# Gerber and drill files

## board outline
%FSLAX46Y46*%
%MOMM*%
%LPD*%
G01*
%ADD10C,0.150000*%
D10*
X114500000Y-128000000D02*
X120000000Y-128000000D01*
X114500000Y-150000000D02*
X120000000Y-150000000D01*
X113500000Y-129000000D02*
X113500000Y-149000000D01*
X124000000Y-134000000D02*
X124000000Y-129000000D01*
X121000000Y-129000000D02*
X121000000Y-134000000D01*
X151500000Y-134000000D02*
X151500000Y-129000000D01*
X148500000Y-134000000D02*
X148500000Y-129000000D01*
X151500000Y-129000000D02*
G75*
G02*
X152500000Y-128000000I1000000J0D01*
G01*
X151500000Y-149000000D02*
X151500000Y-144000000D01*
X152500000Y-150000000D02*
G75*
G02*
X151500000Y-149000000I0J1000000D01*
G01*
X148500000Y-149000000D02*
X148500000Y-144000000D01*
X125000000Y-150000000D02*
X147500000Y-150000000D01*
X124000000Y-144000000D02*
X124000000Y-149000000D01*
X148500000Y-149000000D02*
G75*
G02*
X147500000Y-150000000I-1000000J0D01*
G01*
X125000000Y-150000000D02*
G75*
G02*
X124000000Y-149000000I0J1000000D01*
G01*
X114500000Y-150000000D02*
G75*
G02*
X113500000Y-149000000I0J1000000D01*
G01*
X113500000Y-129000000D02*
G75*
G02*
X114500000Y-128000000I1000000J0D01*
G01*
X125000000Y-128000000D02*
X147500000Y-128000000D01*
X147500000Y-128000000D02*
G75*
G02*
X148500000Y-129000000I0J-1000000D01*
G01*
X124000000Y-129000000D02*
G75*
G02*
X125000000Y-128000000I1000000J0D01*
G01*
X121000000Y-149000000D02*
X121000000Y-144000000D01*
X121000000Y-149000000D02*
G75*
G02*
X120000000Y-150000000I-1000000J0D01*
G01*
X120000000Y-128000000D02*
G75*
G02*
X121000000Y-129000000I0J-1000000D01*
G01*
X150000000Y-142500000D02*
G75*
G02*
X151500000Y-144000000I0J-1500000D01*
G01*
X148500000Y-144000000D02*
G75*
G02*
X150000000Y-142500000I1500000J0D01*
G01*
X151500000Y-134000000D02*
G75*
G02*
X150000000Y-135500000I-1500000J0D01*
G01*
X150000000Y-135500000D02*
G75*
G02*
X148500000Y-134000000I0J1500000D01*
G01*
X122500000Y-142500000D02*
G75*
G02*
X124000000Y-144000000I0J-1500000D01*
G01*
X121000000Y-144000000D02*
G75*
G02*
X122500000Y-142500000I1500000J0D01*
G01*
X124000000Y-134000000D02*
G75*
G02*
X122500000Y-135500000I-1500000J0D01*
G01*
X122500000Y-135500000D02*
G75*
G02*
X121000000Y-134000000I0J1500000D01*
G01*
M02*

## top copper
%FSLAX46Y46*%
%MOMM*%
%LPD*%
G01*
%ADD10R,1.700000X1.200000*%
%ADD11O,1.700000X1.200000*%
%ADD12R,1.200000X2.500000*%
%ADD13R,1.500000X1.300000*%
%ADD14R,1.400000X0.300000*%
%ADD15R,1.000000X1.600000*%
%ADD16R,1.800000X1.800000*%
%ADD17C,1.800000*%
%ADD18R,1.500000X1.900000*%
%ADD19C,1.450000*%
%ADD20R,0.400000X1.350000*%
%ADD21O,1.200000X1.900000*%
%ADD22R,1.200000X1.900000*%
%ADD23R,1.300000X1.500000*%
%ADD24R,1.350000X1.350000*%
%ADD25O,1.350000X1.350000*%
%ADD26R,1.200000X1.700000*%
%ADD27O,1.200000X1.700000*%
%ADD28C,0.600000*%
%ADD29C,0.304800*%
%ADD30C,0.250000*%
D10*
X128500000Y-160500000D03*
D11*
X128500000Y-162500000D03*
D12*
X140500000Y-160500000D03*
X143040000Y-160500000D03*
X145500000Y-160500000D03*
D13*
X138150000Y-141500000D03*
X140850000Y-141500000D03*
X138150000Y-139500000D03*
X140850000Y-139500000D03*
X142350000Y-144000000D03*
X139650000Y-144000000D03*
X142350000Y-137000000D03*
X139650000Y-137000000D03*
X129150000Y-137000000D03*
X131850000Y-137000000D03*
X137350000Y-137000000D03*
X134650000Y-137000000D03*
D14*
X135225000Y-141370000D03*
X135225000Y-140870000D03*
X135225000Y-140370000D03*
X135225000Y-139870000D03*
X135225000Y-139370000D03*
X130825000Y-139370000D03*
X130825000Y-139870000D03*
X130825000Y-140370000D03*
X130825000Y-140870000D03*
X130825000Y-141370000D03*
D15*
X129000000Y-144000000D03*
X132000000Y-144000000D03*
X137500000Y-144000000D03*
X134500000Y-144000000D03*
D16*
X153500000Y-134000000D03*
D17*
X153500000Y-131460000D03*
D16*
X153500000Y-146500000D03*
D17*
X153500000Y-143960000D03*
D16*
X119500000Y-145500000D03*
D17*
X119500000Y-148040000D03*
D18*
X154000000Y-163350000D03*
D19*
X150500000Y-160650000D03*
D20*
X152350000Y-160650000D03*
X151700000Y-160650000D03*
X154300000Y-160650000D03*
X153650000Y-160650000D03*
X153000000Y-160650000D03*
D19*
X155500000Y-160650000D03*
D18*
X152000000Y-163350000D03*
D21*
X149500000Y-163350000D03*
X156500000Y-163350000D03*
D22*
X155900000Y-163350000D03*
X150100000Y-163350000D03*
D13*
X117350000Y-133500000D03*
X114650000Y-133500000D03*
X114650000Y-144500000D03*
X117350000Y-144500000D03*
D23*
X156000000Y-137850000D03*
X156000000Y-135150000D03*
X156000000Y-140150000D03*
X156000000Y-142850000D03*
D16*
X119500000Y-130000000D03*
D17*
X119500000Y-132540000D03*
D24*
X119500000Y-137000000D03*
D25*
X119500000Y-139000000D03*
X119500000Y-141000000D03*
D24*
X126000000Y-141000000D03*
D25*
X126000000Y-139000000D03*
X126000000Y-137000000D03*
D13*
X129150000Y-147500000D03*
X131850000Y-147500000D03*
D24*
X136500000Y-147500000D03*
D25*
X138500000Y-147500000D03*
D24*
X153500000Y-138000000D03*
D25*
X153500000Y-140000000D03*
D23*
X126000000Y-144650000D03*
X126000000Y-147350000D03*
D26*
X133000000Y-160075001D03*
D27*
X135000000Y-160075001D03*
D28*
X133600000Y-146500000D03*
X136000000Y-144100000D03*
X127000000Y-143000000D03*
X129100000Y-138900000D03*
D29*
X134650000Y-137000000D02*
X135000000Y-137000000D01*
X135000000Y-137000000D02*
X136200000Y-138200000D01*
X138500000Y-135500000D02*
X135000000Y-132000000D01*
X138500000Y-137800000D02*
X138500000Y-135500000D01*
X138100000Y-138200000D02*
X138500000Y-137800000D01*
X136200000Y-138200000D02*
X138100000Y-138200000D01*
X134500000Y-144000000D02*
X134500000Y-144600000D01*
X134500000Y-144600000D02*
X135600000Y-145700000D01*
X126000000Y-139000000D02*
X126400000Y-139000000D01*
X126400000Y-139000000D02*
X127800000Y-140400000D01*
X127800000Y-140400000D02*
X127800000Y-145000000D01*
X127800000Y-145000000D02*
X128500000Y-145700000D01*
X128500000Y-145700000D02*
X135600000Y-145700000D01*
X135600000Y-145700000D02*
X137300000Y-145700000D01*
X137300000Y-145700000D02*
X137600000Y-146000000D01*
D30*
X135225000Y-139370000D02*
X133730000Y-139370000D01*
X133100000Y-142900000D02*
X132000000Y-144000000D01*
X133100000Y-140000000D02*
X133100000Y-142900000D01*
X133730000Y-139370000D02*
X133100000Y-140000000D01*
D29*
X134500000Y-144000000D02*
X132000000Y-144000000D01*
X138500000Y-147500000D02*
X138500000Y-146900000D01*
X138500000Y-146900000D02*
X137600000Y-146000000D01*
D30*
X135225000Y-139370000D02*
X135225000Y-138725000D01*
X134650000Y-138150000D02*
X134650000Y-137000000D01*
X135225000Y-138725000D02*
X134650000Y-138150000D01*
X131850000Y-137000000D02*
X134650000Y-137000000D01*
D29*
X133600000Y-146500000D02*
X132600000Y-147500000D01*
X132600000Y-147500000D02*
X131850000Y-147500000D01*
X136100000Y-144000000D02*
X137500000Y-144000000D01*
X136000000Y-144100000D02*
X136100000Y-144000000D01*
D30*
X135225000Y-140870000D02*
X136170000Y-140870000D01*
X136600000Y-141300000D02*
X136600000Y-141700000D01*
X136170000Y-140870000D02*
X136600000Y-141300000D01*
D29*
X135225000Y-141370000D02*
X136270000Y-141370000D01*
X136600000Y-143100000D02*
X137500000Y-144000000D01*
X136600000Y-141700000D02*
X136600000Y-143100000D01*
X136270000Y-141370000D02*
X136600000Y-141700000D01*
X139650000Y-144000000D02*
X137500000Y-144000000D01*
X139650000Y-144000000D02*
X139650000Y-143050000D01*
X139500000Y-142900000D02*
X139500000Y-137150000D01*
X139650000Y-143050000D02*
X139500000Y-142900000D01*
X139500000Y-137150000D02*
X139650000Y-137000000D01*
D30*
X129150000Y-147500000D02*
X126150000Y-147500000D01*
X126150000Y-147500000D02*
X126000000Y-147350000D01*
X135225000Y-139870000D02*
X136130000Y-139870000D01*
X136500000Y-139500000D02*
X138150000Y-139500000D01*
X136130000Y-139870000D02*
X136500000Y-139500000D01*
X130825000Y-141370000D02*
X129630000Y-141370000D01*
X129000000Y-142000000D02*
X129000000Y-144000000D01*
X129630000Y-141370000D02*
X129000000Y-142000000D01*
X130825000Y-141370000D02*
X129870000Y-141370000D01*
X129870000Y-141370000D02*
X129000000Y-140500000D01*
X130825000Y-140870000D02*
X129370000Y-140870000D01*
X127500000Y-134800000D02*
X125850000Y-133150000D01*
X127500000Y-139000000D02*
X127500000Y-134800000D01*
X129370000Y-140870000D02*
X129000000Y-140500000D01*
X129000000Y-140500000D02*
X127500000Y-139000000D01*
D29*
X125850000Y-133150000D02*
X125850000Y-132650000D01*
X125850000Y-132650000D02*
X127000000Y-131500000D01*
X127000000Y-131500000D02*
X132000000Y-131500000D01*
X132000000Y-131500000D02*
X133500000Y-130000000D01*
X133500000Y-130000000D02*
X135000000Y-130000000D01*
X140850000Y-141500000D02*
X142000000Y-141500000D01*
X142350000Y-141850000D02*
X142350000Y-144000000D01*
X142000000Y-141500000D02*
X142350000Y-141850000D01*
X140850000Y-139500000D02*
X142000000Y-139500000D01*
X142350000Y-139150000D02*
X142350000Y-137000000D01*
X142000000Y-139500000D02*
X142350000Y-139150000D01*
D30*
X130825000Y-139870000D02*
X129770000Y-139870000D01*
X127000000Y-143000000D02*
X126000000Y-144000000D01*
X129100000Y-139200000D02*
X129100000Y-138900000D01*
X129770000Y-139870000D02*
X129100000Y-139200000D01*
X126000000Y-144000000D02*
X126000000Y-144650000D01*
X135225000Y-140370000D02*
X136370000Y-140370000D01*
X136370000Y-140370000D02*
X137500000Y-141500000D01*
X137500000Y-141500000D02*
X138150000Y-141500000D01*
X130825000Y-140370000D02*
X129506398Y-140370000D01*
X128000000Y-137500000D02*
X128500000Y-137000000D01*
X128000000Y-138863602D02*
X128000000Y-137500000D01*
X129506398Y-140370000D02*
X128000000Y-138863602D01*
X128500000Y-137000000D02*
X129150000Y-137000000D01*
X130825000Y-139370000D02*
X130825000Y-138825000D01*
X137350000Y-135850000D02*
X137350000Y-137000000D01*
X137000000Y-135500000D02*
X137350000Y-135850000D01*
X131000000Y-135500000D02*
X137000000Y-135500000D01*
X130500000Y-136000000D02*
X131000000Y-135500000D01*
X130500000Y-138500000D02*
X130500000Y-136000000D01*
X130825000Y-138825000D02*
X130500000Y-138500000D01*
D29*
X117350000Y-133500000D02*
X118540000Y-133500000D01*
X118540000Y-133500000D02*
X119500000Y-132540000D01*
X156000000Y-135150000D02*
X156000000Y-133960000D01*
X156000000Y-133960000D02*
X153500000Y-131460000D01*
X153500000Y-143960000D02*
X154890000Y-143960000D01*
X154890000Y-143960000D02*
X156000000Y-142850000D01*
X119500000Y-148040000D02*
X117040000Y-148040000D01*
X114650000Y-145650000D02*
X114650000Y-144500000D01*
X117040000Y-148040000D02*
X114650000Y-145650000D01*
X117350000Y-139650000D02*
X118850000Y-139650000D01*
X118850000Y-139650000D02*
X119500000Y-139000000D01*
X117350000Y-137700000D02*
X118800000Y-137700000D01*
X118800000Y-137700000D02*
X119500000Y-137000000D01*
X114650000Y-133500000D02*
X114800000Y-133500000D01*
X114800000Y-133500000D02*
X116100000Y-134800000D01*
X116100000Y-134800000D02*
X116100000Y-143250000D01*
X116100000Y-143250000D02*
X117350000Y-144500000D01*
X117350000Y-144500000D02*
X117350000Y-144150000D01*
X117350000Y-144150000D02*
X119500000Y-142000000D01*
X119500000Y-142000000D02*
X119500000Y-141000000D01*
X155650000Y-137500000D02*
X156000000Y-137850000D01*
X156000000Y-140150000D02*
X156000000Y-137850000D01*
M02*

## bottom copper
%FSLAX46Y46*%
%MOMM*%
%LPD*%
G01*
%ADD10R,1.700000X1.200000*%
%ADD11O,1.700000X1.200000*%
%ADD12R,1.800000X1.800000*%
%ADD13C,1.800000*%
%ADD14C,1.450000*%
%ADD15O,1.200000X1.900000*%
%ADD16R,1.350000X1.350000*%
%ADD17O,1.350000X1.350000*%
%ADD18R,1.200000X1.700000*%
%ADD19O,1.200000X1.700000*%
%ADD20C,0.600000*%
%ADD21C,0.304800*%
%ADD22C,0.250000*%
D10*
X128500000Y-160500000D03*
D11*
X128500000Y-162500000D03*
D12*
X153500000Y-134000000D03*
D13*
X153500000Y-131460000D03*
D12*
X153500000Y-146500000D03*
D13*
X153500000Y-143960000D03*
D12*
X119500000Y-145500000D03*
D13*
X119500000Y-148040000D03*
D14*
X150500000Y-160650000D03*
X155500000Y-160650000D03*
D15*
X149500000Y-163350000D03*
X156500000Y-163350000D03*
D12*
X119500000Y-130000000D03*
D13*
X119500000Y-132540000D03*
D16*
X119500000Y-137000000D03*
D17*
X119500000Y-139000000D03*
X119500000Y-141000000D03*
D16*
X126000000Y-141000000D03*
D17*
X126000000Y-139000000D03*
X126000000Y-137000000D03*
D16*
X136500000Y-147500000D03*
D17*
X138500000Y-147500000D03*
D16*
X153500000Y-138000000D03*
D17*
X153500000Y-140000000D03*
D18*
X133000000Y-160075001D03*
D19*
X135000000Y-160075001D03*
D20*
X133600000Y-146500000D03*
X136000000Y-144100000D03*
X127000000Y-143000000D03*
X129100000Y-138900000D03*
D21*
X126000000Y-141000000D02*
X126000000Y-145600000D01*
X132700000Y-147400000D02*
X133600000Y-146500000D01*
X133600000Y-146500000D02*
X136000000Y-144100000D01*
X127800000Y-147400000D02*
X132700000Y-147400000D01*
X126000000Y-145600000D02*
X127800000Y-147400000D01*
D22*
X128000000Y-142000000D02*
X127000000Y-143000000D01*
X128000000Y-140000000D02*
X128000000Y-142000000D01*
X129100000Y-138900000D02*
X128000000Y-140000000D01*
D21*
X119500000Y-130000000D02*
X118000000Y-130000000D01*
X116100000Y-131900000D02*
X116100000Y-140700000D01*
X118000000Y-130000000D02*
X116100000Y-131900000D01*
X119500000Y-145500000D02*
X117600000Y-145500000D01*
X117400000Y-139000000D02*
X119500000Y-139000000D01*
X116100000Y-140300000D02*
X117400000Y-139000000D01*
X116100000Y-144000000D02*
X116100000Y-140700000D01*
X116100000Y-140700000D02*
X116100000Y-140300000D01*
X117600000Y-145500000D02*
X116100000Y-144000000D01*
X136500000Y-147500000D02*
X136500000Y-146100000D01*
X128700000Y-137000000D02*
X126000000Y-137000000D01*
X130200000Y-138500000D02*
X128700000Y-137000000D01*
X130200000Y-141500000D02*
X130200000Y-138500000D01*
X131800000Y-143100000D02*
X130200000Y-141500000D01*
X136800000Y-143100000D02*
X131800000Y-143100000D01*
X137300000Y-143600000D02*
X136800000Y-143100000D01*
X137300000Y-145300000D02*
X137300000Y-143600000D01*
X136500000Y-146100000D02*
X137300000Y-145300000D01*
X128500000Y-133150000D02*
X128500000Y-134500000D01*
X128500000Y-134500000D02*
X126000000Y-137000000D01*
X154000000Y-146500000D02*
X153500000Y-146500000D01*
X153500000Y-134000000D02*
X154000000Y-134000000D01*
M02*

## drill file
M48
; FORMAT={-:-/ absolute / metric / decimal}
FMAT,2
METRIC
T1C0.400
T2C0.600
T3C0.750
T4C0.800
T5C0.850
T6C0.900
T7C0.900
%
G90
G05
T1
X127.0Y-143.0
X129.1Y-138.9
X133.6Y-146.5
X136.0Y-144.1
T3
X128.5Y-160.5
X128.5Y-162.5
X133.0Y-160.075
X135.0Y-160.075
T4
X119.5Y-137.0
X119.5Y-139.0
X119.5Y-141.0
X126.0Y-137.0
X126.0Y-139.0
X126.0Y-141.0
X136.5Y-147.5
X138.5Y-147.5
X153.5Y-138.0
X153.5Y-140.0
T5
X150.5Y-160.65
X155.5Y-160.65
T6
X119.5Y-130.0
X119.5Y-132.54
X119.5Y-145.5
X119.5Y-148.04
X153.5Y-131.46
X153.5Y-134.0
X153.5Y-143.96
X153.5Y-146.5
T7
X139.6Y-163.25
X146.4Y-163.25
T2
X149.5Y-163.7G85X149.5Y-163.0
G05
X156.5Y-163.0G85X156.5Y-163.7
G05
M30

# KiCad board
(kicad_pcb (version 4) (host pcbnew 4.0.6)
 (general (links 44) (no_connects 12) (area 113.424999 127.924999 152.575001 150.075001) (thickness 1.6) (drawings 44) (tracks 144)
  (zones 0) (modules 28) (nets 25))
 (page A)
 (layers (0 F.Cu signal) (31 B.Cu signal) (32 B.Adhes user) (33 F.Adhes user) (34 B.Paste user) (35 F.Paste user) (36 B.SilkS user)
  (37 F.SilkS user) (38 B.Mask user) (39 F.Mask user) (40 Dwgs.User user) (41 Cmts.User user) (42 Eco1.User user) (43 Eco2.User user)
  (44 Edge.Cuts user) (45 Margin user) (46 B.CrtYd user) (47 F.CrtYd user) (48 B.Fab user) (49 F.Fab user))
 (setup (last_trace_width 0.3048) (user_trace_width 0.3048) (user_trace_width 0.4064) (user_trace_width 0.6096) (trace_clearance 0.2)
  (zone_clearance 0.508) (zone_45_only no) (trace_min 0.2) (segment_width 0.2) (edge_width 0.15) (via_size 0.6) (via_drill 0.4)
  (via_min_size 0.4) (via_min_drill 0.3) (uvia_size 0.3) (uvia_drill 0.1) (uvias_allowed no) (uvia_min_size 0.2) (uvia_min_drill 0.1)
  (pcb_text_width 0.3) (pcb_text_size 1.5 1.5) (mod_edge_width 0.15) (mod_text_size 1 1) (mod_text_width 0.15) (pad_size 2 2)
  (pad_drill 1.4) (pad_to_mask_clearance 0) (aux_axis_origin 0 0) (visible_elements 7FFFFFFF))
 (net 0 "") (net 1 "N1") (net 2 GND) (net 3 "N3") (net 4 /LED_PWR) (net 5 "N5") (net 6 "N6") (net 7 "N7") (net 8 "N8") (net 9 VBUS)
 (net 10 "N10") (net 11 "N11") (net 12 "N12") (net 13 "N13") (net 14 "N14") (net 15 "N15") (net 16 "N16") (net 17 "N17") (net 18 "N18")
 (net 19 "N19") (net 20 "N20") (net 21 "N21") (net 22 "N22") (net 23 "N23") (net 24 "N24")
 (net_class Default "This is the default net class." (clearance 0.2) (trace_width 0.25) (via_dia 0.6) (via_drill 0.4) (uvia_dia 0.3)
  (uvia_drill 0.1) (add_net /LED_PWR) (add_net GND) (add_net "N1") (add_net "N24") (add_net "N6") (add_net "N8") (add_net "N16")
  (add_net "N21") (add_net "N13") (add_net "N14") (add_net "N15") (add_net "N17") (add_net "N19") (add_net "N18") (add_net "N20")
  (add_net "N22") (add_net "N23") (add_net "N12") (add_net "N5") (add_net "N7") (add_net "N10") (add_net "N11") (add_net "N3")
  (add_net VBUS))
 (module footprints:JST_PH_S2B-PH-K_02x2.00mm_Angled (layer F.Cu) (at 128.5 160.5 270)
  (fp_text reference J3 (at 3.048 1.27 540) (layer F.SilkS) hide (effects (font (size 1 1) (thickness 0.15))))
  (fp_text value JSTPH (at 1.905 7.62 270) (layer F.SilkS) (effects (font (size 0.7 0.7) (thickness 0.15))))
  (pad 1 thru_hole rect (at 0 0 270) (size 1.2 1.7) (drill 0.75) (layers *.Cu *.Mask) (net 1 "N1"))
  (pad 2 thru_hole oval (at 2 0 270) (size 1.2 1.7) (drill 0.75) (layers *.Cu *.Mask) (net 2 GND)))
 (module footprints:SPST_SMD (layer F.Cu) (at 143 160.5)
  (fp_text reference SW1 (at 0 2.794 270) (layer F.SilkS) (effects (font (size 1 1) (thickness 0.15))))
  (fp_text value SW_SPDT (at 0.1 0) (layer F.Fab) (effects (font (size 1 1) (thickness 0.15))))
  (pad "" np_thru_hole circle (at 3.4 2.75) (size 0.9 0.9) (drill 0.9) (layers *.Cu *.Mask))
  (pad 1 smd rect (at -2.5 0) (size 1.2 2.5) (layers F.Cu F.Paste F.Mask) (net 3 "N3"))
  (pad 2 smd rect (at 0.04 0) (size 1.2 2.5) (layers F.Cu F.Paste F.Mask) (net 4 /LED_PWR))
  (pad 3 smd rect (at 2.5 0) (size 1.2 2.5) (layers F.Cu F.Paste F.Mask) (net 1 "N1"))
  (pad "" np_thru_hole circle (at -3.4 2.75) (size 0.9 0.9) (drill 0.9) (layers *.Cu *.Mask)))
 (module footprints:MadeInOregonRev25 (layer F.Cu) (at 158 109.5)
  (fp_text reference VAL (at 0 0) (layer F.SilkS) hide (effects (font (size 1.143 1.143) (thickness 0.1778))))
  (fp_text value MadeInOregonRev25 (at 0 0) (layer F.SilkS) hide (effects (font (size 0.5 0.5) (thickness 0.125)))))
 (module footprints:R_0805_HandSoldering (layer F.Cu) (at 139.5 141.5)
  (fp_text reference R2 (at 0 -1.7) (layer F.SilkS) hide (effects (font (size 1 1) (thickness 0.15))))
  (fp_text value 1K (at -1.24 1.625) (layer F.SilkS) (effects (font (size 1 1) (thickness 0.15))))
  (pad 1 smd rect (at -1.35 0) (size 1.5 1.3) (layers F.Cu F.Paste F.Mask) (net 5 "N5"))
  (pad 2 smd rect (at 1.35 0) (size 1.5 1.3) (layers F.Cu F.Paste F.Mask) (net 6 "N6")))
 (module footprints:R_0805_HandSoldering (layer F.Cu) (at 139.5 139.5)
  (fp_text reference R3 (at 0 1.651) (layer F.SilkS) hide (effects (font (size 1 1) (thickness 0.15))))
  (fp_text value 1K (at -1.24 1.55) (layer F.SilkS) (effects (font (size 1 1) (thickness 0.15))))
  (pad 1 smd rect (at -1.35 0) (size 1.5 1.3) (layers F.Cu F.Paste F.Mask) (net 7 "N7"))
  (pad 2 smd rect (at 1.35 0) (size 1.5 1.3) (layers F.Cu F.Paste F.Mask) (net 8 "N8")))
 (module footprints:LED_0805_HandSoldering (layer F.Cu) (at 141 144 180)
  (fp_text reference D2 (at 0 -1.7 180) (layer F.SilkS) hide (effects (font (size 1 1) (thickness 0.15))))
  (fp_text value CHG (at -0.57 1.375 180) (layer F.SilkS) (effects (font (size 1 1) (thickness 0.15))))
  (pad 1 smd rect (at -1.35 0 180) (size 1.5 1.3) (layers F.Cu F.Paste F.Mask) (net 6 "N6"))
  (pad 2 smd rect (at 1.35 0 180) (size 1.5 1.3) (layers F.Cu F.Paste F.Mask) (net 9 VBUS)))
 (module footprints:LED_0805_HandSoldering (layer F.Cu) (at 141 137 180)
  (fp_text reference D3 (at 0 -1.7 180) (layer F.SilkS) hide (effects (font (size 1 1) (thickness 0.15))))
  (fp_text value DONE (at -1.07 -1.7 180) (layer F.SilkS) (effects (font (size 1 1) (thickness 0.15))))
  (pad 1 smd rect (at -1.35 0 180) (size 1.5 1.3) (layers F.Cu F.Paste F.Mask) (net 8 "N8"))
  (pad 2 smd rect (at 1.35 0 180) (size 1.5 1.3) (layers F.Cu F.Paste F.Mask) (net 9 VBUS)))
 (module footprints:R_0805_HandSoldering (layer F.Cu) (at 130.5 137)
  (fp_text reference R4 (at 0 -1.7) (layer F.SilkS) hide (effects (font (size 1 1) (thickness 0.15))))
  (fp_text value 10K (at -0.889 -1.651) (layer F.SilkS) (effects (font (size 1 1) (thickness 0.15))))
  (pad 1 smd rect (at -1.35 0) (size 1.5 1.3) (layers F.Cu F.Paste F.Mask) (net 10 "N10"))
  (pad 2 smd rect (at 1.35 0) (size 1.5 1.3) (layers F.Cu F.Paste F.Mask) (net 2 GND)))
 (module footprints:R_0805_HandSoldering (layer F.Cu) (at 136 137 180)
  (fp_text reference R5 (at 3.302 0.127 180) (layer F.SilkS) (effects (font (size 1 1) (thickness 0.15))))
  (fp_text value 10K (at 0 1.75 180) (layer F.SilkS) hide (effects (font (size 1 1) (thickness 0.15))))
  (pad 1 smd rect (at -1.35 0 180) (size 1.5 1.3) (layers F.Cu F.Paste F.Mask) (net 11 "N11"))
  (pad 2 smd rect (at 1.35 0 180) (size 1.5 1.3) (layers F.Cu F.Paste F.Mask) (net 2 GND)))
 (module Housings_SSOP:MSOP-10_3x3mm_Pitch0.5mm (layer F.Cu) (at 133.025 140.37 180)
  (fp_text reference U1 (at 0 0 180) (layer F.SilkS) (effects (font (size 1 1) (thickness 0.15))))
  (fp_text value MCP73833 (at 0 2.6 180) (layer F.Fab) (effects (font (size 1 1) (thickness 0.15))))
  (pad 1 smd rect (at -2.2 -1 180) (size 1.4 0.3) (layers F.Cu F.Paste F.Mask) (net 9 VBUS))
  (pad 2 smd rect (at -2.2 -0.5 180) (size 1.4 0.3) (layers F.Cu F.Paste F.Mask) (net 9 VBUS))
  (pad 3 smd rect (at -2.2 0 180) (size 1.4 0.3) (layers F.Cu F.Paste F.Mask) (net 5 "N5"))
  (pad 4 smd rect (at -2.2 0.5 180) (size 1.4 0.3) (layers F.Cu F.Paste F.Mask) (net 7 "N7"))
  (pad 5 smd rect (at -2.2 1 180) (size 1.4 0.3) (layers F.Cu F.Paste F.Mask) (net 2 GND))
  (pad 6 smd rect (at 2.2 1 180) (size 1.4 0.3) (layers F.Cu F.Paste F.Mask) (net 11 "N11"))
  (pad 7 smd rect (at 2.2 0.5 180) (size 1.4 0.3) (layers F.Cu F.Paste F.Mask) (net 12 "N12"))
  (pad 8 smd rect (at 2.2 0 180) (size 1.4 0.3) (layers F.Cu F.Paste F.Mask) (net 10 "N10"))
  (pad 9 smd rect (at 2.2 -0.5 180) (size 1.4 0.3) (layers F.Cu F.Paste F.Mask) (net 1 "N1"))
  (pad 10 smd rect (at 2.2 -1 180) (size 1.4 0.3) (layers F.Cu F.Paste F.Mask) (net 1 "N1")))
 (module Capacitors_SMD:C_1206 (layer F.Cu) (at 130.5 144)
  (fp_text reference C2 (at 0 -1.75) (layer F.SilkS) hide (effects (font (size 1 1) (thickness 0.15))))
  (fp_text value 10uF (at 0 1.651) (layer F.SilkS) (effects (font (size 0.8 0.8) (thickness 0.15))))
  (pad 1 smd rect (at -1.5 0) (size 1 1.6) (layers F.Cu F.Paste F.Mask) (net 1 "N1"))
  (pad 2 smd rect (at 1.5 0) (size 1 1.6) (layers F.Cu F.Paste F.Mask) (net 2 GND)))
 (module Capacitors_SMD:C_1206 (layer F.Cu) (at 136 144 180)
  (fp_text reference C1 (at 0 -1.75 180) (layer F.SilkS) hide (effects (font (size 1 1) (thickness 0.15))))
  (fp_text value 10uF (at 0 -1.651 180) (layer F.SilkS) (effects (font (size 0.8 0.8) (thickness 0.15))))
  (pad 1 smd rect (at -1.5 0 180) (size 1 1.6) (layers F.Cu F.Paste F.Mask) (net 9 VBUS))
  (pad 2 smd rect (at 1.5 0 180) (size 1 1.6) (layers F.Cu F.Paste F.Mask) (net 2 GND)))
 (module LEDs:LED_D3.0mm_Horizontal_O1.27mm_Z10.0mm (layer F.Cu) (at 153.5 134 90)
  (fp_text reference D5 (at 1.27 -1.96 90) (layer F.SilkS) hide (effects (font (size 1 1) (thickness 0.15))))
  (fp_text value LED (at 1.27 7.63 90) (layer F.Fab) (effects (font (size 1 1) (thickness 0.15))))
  (pad 1 thru_hole rect (at 0 0 90) (size 1.8 1.8) (drill 0.9) (layers *.Cu *.Mask) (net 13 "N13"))
  (pad 2 thru_hole circle (at 2.54 0 90) (size 1.8 1.8) (drill 0.9) (layers *.Cu *.Mask) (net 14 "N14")))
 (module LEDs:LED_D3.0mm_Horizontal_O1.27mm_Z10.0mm (layer F.Cu) (at 153.5 146.5 90)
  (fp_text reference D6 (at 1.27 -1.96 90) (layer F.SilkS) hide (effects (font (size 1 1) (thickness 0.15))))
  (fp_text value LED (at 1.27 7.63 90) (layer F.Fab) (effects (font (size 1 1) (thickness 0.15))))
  (pad 1 thru_hole rect (at 0 0 90) (size 1.8 1.8) (drill 0.9) (layers *.Cu *.Mask) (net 13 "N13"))
  (pad 2 thru_hole circle (at 2.54 0 90) (size 1.8 1.8) (drill 0.9) (layers *.Cu *.Mask) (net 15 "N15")))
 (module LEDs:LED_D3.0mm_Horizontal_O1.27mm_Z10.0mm (layer F.Cu) (at 119.5 145.5 270)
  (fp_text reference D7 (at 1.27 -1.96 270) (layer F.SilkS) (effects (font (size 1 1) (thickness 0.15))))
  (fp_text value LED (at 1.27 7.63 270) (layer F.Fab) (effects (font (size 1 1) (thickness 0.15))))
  (pad 1 thru_hole rect (at 0 0 270) (size 1.8 1.8) (drill 0.9) (layers *.Cu *.Mask) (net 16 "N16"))
  (pad 2 thru_hole circle (at 2.54 0 270) (size 1.8 1.8) (drill 0.9) (layers *.Cu *.Mask) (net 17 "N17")))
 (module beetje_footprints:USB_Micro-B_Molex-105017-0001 (layer F.Cu) (at 153 163)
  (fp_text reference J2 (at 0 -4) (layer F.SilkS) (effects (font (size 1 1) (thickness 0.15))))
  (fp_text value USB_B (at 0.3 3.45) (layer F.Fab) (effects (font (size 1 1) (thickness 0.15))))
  (pad 6 smd rect (at 1 0.35) (size 1.5 1.9) (layers F.Cu F.Paste F.Mask))
  (pad 6 thru_hole circle (at -2.5 -2.35) (size 1.45 1.45) (drill 0.85) (layers *.Cu *.Mask))
  (pad 2 smd rect (at -0.65 -2.35) (size 0.4 1.35) (layers F.Cu F.Paste F.Mask) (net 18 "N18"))
  (pad 1 smd rect (at -1.3 -2.35) (size 0.4 1.35) (layers F.Cu F.Paste F.Mask) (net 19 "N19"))
  (pad 5 smd rect (at 1.3 -2.35) (size 0.4 1.35) (layers F.Cu F.Paste F.Mask) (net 16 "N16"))
  (pad 4 smd rect (at 0.65 -2.35) (size 0.4 1.35) (layers F.Cu F.Paste F.Mask) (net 16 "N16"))
  (pad 3 smd rect (at 0 -2.35) (size 0.4 1.35) (layers F.Cu F.Paste F.Mask) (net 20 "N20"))
  (pad 6 thru_hole circle (at 2.5 -2.35) (size 1.45 1.45) (drill 0.85) (layers *.Cu *.Mask))
  (pad 6 smd rect (at -1 0.35) (size 1.5 1.9) (layers F.Cu F.Paste F.Mask))
  (pad 6 thru_hole oval (at -3.5 0.35 180) (size 1.2 1.9) (drill oval 0.6 1.3) (layers *.Cu *.Mask))
  (pad 6 thru_hole oval (at 3.5 0.35) (size 1.2 1.9) (drill oval 0.6 1.3) (layers *.Cu *.Mask))
  (pad 6 smd rect (at 2.9 0.35) (size 1.2 1.9) (layers F.Cu F.Mask))
  (pad 6 smd rect (at -2.9 0.35) (size 1.2 1.9) (layers F.Cu F.Mask)))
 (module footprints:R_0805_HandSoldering (layer F.Cu) (at 116 133.5 180)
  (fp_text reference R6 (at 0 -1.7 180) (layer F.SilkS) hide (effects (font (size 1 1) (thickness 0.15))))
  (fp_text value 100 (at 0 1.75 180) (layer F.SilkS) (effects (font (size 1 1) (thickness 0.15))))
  (pad 1 smd rect (at -1.35 0 180) (size 1.5 1.3) (layers F.Cu F.Paste F.Mask) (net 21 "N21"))
  (pad 2 smd rect (at 1.35 0 180) (size 1.5 1.3) (layers F.Cu F.Paste F.Mask) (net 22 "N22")))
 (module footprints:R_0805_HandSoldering (layer F.Cu) (at 116 144.5)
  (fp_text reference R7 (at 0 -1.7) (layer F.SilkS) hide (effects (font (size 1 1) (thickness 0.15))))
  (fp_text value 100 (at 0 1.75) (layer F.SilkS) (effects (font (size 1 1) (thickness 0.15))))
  (pad 1 smd rect (at -1.35 0) (size 1.5 1.3) (layers F.Cu F.Paste F.Mask) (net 17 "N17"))
  (pad 2 smd rect (at 1.35 0) (size 1.5 1.3) (layers F.Cu F.Paste F.Mask) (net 22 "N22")))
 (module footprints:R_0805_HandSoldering (layer F.Cu) (at 156 136.5 90)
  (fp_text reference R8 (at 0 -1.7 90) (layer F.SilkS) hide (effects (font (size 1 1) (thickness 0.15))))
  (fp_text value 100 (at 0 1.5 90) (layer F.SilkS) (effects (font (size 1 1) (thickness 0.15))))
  (pad 1 smd rect (at -1.35 0 90) (size 1.5 1.3) (layers F.Cu F.Paste F.Mask) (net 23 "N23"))
  (pad 2 smd rect (at 1.35 0 90) (size 1.5 1.3) (layers F.Cu F.Paste F.Mask) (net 14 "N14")))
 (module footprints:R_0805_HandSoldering (layer F.Cu) (at 156 141.5 270)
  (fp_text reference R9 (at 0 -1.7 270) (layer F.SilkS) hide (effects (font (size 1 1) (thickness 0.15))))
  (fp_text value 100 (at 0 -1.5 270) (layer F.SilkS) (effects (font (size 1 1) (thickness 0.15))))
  (pad 1 smd rect (at -1.35 0 270) (size 1.5 1.3) (layers F.Cu F.Paste F.Mask) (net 23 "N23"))
  (pad 2 smd rect (at 1.35 0 270) (size 1.5 1.3) (layers F.Cu F.Paste F.Mask) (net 15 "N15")))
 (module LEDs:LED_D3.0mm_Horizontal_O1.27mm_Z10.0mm (layer F.Cu) (at 119.5 130 270)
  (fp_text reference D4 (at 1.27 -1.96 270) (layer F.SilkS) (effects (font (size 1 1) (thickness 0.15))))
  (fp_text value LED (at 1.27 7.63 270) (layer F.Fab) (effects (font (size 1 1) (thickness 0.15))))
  (pad 1 thru_hole rect (at 0 0 270) (size 1.8 1.8) (drill 0.9) (layers *.Cu *.Mask) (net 16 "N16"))
  (pad 2 thru_hole circle (at 2.54 0 270) (size 1.8 1.8) (drill 0.9) (layers *.Cu *.Mask) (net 21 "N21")))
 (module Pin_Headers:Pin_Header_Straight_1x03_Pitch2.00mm (layer F.Cu) (at 119.5 137)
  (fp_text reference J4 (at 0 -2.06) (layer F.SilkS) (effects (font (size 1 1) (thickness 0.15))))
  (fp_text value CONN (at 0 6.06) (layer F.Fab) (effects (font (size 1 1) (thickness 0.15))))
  (pad 1 thru_hole rect (at 0 0) (size 1.35 1.35) (drill 0.8) (layers *.Cu *.Mask) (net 19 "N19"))
  (pad 2 thru_hole oval (at 0 2) (size 1.35 1.35) (drill 0.8) (layers *.Cu *.Mask) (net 16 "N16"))
  (pad 3 thru_hole oval (at 0 4) (size 1.35 1.35) (drill 0.8) (layers *.Cu *.Mask) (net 22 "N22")))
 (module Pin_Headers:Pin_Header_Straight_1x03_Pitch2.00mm (layer F.Cu) (at 126 141 180)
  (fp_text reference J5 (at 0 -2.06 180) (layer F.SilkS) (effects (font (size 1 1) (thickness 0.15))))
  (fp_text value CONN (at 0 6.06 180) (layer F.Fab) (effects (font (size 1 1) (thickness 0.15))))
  (pad 1 thru_hole rect (at 0 0 180) (size 1.35 1.35) (drill 0.8) (layers *.Cu *.Mask) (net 9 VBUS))
  (pad 2 thru_hole oval (at 0 2 180) (size 1.35 1.35) (drill 0.8) (layers *.Cu *.Mask) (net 2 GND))
  (pad 3 thru_hole oval (at 0 4 180) (size 1.35 1.35) (drill 0.8) (layers *.Cu *.Mask) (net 4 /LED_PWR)))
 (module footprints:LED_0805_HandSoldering (layer F.Cu) (at 130.5 147.5)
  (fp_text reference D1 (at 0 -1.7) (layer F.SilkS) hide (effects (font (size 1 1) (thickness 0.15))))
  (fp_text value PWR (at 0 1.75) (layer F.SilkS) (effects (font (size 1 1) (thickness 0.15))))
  (pad 1 smd rect (at -1.35 0) (size 1.5 1.3) (layers F.Cu F.Paste F.Mask) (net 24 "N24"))
  (pad 2 smd rect (at 1.35 0) (size 1.5 1.3) (layers F.Cu F.Paste F.Mask) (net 9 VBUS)))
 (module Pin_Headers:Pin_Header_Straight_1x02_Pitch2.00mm (layer F.Cu) (at 136.5 147.5 90)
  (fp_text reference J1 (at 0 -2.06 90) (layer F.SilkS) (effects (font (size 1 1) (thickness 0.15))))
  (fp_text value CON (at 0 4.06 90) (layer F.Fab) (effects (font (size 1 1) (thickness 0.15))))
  (pad 1 thru_hole rect (at 0 0 90) (size 1.35 1.35) (drill 0.8) (layers *.Cu *.Mask) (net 4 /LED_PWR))
  (pad 2 thru_hole oval (at 0 2 90) (size 1.35 1.35) (drill 0.8) (layers *.Cu *.Mask) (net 2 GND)))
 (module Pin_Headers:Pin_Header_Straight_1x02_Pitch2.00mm (layer F.Cu) (at 153.5 138)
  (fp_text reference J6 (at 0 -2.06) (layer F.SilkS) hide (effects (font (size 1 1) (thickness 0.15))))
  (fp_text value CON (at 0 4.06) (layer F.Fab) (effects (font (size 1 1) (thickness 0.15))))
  (pad 1 thru_hole rect (at 0 0) (size 1.35 1.35) (drill 0.8) (layers *.Cu *.Mask) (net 23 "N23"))
  (pad 2 thru_hole oval (at 0 2) (size 1.35 1.35) (drill 0.8) (layers *.Cu *.Mask) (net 13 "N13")))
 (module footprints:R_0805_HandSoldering (layer F.Cu) (at 126 146 270)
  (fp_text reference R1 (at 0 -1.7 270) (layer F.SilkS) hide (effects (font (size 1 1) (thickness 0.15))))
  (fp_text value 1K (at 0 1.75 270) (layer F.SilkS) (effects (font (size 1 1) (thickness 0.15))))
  (pad 1 smd rect (at -1.35 0 270) (size 1.5 1.3) (layers F.Cu F.Paste F.Mask) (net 12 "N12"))
  (pad 2 smd rect (at 1.35 0 270) (size 1.5 1.3) (layers F.Cu F.Paste F.Mask) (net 24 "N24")))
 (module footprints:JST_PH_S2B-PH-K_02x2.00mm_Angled (layer F.Cu) (at 133 160.075001)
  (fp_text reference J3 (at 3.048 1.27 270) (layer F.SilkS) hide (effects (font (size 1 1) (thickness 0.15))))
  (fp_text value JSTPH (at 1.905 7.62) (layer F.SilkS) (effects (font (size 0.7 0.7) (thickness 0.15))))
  (pad 1 thru_hole rect (at 0 0) (size 1.2 1.7) (drill 0.75) (layers *.Cu *.Mask) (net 1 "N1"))
  (pad 2 thru_hole oval (at 2 0) (size 1.2 1.7) (drill 0.75) (layers *.Cu *.Mask) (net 2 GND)))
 (gr_line (start 114.5 128) (end 120 128) (angle 90) (layer Edge.Cuts) (width 0.15))
 (gr_line (start 114.5 150) (end 120 150) (angle 90) (layer Edge.Cuts) (width 0.15))
 (gr_line (start 113.5 129) (end 113.5 149) (angle 90) (layer Edge.Cuts) (width 0.15))
 (gr_line (start 124 134) (end 124 129) (angle 90) (layer Edge.Cuts) (width 0.15))
 (gr_line (start 121 129) (end 121 134) (angle 90) (layer Edge.Cuts) (width 0.15))
 (gr_line (start 151.5 134) (end 151.5 129) (angle 90) (layer Edge.Cuts) (width 0.15))
 (gr_line (start 148.5 134) (end 148.5 129) (angle 90) (layer Edge.Cuts) (width 0.15))
 (gr_arc (start 152.5 129) (end 151.5 129) (angle 90) (layer Edge.Cuts) (width 0.15))
 (gr_line (start 151.5 149) (end 151.5 144) (angle 90) (layer Edge.Cuts) (width 0.15))
 (gr_arc (start 152.5 149) (end 152.5 150) (angle 90) (layer Edge.Cuts) (width 0.15))
 (gr_line (start 148.5 149) (end 148.5 144) (angle 90) (layer Edge.Cuts) (width 0.15))
 (gr_line (start 125 150) (end 147.5 150) (angle 90) (layer Edge.Cuts) (width 0.15))
 (gr_line (start 124 144) (end 124 149) (angle 90) (layer Edge.Cuts) (width 0.15))
 (gr_arc (start 147.5 149) (end 148.5 149) (angle 90) (layer Edge.Cuts) (width 0.15))
 (gr_arc (start 125 149) (end 125 150) (angle 90) (layer Edge.Cuts) (width 0.15))
 (gr_arc (start 114.5 149) (end 114.5 150) (angle 90) (layer Edge.Cuts) (width 0.15))
 (gr_arc (start 114.5 129) (end 113.5 129) (angle 90) (layer Edge.Cuts) (width 0.15))
 (gr_line (start 125 128) (end 147.5 128) (angle 90) (layer Edge.Cuts) (width 0.15))
 (gr_arc (start 147.5 129) (end 147.5 128) (angle 90) (layer Edge.Cuts) (width 0.15))
 (gr_arc (start 125 129) (end 124 129) (angle 90) (layer Edge.Cuts) (width 0.15))
 (gr_line (start 121 149) (end 121 144) (angle 90) (layer Edge.Cuts) (width 0.15))
 (gr_arc (start 120 149) (end 121 149) (angle 90) (layer Edge.Cuts) (width 0.15))
 (gr_arc (start 120 129) (end 120 128) (angle 90) (layer Edge.Cuts) (width 0.15))
 (gr_arc (start 150 144) (end 150 142.5) (angle 90) (layer Edge.Cuts) (width 0.15))
 (gr_arc (start 150 144) (end 148.5 144) (angle 90) (layer Edge.Cuts) (width 0.15))
 (gr_arc (start 150 134) (end 151.5 134) (angle 90) (layer Edge.Cuts) (width 0.15))
 (gr_arc (start 150 134) (end 150 135.5) (angle 90) (layer Edge.Cuts) (width 0.15))
 (gr_arc (start 122.5 144) (end 122.5 142.5) (angle 90) (layer Edge.Cuts) (width 0.15))
 (gr_arc (start 122.5 144) (end 121 144) (angle 90) (layer Edge.Cuts) (width 0.15))
 (gr_arc (start 122.5 134) (end 124 134) (angle 90) (layer Edge.Cuts) (width 0.15))
 (gr_arc (start 122.5 134) (end 122.5 135.5) (angle 90) (layer Edge.Cuts) (width 0.15))
 (segment (start 134.65 137) (end 135 137) (width 0.3048) (layer F.Cu) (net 2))
 (segment (start 135 137) (end 136.2 138.2) (width 0.3048) (layer F.Cu) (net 2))
 (segment (start 138.5 135.5) (end 135 132) (width 0.3048) (layer F.Cu) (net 2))
 (segment (start 138.5 137.8) (end 138.5 135.5) (width 0.3048) (layer F.Cu) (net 2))
 (segment (start 138.1 138.2) (end 138.5 137.8) (width 0.3048) (layer F.Cu) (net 2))
 (segment (start 136.2 138.2) (end 138.1 138.2) (width 0.3048) (layer F.Cu) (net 2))
 (segment (start 134.5 144) (end 134.5 144.6) (width 0.3048) (layer F.Cu) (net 2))
 (segment (start 134.5 144.6) (end 135.6 145.7) (width 0.3048) (layer F.Cu) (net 2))
 (segment (start 126 139) (end 126.4 139) (width 0.3048) (layer F.Cu) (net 2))
 (segment (start 126.4 139) (end 127.8 140.4) (width 0.3048) (layer F.Cu) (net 2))
 (segment (start 127.8 140.4) (end 127.8 145) (width 0.3048) (layer F.Cu) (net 2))
 (segment (start 127.8 145) (end 128.5 145.7) (width 0.3048) (layer F.Cu) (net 2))
 (segment (start 128.5 145.7) (end 135.6 145.7) (width 0.3048) (layer F.Cu) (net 2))
 (segment (start 135.6 145.7) (end 137.3 145.7) (width 0.3048) (layer F.Cu) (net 2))
 (segment (start 137.3 145.7) (end 137.6 146) (width 0.3048) (layer F.Cu) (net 2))
 (segment (start 135.225 139.37) (end 133.73 139.37) (width 0.25) (layer F.Cu) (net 2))
 (segment (start 133.1 142.9) (end 132 144) (width 0.25) (layer F.Cu) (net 2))
 (segment (start 133.1 140) (end 133.1 142.9) (width 0.25) (layer F.Cu) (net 2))
 (segment (start 133.73 139.37) (end 133.1 140) (width 0.25) (layer F.Cu) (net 2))
 (segment (start 134.5 144) (end 132 144) (width 0.3048) (layer F.Cu) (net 2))
 (segment (start 138.5 147.5) (end 138.5 146.9) (width 0.3048) (layer F.Cu) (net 2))
 (segment (start 138.5 146.9) (end 137.6 146) (width 0.3048) (layer F.Cu) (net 2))
 (segment (start 135.225 139.37) (end 135.225 138.725) (width 0.25) (layer F.Cu) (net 2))
 (segment (start 134.65 138.15) (end 134.65 137) (width 0.25) (layer F.Cu) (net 2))
 (segment (start 135.225 138.725) (end 134.65 138.15) (width 0.25) (layer F.Cu) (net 2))
 (segment (start 131.85 137) (end 134.65 137) (width 0.25) (layer F.Cu) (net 2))
 (via (at 133.6 146.5) (size 0.6) (drill 0.4) (layers F.Cu B.Cu) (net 9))
 (segment (start 133.6 146.5) (end 132.6 147.5) (width 0.3048) (layer F.Cu) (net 9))
 (segment (start 132.6 147.5) (end 131.85 147.5) (width 0.3048) (layer F.Cu) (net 9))
 (segment (start 126 141) (end 126 145.6) (width 0.3048) (layer B.Cu) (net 9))
 (segment (start 136.1 144) (end 137.5 144) (width 0.3048) (layer F.Cu) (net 9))
 (segment (start 136 144.1) (end 136.1 144) (width 0.3048) (layer F.Cu) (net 9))
 (via (at 136 144.1) (size 0.6) (drill 0.4) (layers F.Cu B.Cu) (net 9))
 (segment (start 132.7 147.4) (end 133.6 146.5) (width 0.3048) (layer B.Cu) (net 9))
 (segment (start 133.6 146.5) (end 136 144.1) (width 0.3048) (layer B.Cu) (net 9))
 (segment (start 127.8 147.4) (end 132.7 147.4) (width 0.3048) (layer B.Cu) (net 9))
 (segment (start 126 145.6) (end 127.8 147.4) (width 0.3048) (layer B.Cu) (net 9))
 (segment (start 135.225 140.87) (end 136.17 140.87) (width 0.25) (layer F.Cu) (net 9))
 (segment (start 136.6 141.3) (end 136.6 141.7) (width 0.25) (layer F.Cu) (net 9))
 (segment (start 136.17 140.87) (end 136.6 141.3) (width 0.25) (layer F.Cu) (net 9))
 (segment (start 135.225 141.37) (end 136.27 141.37) (width 0.3048) (layer F.Cu) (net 9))
 (segment (start 136.6 143.1) (end 137.5 144) (width 0.3048) (layer F.Cu) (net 9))
 (segment (start 136.6 141.7) (end 136.6 143.1) (width 0.3048) (layer F.Cu) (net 9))
 (segment (start 136.27 141.37) (end 136.6 141.7) (width 0.3048) (layer F.Cu) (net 9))
 (segment (start 139.65 144) (end 137.5 144) (width 0.3048) (layer F.Cu) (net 9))
 (segment (start 139.65 144) (end 139.65 143.05) (width 0.3048) (layer F.Cu) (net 9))
 (segment (start 139.5 142.9) (end 139.5 137.15) (width 0.3048) (layer F.Cu) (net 9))
 (segment (start 139.65 143.05) (end 139.5 142.9) (width 0.3048) (layer F.Cu) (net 9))
 (segment (start 139.5 137.15) (end 139.65 137) (width 0.3048) (layer F.Cu) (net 9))
 (segment (start 129.15 147.5) (end 126.15 147.5) (width 0.25) (layer F.Cu) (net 24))
 (segment (start 126.15 147.5) (end 126 147.35) (width 0.25) (layer F.Cu) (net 24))
 (segment (start 135.225 139.87) (end 136.13 139.87) (width 0.25) (layer F.Cu) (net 7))
 (segment (start 136.5 139.5) (end 138.15 139.5) (width 0.25) (layer F.Cu) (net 7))
 (segment (start 136.13 139.87) (end 136.5 139.5) (width 0.25) (layer F.Cu) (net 7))
 (segment (start 130.825 141.37) (end 129.63 141.37) (width 0.25) (layer F.Cu) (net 1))
 (segment (start 129 142) (end 129 144) (width 0.25) (layer F.Cu) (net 1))
 (segment (start 129.63 141.37) (end 129 142) (width 0.25) (layer F.Cu) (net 1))
 (segment (start 130.825 141.37) (end 129.87 141.37) (width 0.25) (layer F.Cu) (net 1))
 (segment (start 129.87 141.37) (end 129 140.5) (width 0.25) (layer F.Cu) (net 1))
 (segment (start 130.825 140.87) (end 129.37 140.87) (width 0.25) (layer F.Cu) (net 1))
 (segment (start 127.5 134.8) (end 125.85 133.15) (width 0.25) (layer F.Cu) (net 1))
 (segment (start 127.5 139) (end 127.5 134.8) (width 0.25) (layer F.Cu) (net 1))
 (segment (start 129.37 140.87) (end 129 140.5) (width 0.25) (layer F.Cu) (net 1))
 (segment (start 129 140.5) (end 127.5 139) (width 0.25) (layer F.Cu) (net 1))
 (segment (start 125.85 133.15) (end 125.85 132.65) (width 0.3048) (layer F.Cu) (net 1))
 (segment (start 125.85 132.65) (end 127 131.5) (width 0.3048) (layer F.Cu) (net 1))
 (segment (start 127 131.5) (end 132 131.5) (width 0.3048) (layer F.Cu) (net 1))
 (segment (start 132 131.5) (end 133.5 130) (width 0.3048) (layer F.Cu) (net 1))
 (segment (start 133.5 130) (end 135 130) (width 0.3048) (layer F.Cu) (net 1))
 (segment (start 140.85 141.5) (end 142 141.5) (width 0.3048) (layer F.Cu) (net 6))
 (segment (start 142.35 141.85) (end 142.35 144) (width 0.3048) (layer F.Cu) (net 6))
 (segment (start 142 141.5) (end 142.35 141.85) (width 0.3048) (layer F.Cu) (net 6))
 (segment (start 140.85 139.5) (end 142 139.5) (width 0.3048) (layer F.Cu) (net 8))
 (segment (start 142.35 139.15) (end 142.35 137) (width 0.3048) (layer F.Cu) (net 8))
 (segment (start 142 139.5) (end 142.35 139.15) (width 0.3048) (layer F.Cu) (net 8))
 (segment (start 130.825 139.87) (end 129.77 139.87) (width 0.25) (layer F.Cu) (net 12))
 (segment (start 127 143) (end 126 144) (width 0.25) (layer F.Cu) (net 12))
 (via (at 127 143) (size 0.6) (drill 0.4) (layers F.Cu B.Cu) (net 12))
 (segment (start 128 142) (end 127 143) (width 0.25) (layer B.Cu) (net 12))
 (segment (start 128 140) (end 128 142) (width 0.25) (layer B.Cu) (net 12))
 (segment (start 129.1 138.9) (end 128 140) (width 0.25) (layer B.Cu) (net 12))
 (via (at 129.1 138.9) (size 0.6) (drill 0.4) (layers F.Cu B.Cu) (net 12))
 (segment (start 129.1 139.2) (end 129.1 138.9) (width 0.25) (layer F.Cu) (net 12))
 (segment (start 129.77 139.87) (end 129.1 139.2) (width 0.25) (layer F.Cu) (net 12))
 (segment (start 126 144) (end 126 144.65) (width 0.25) (layer F.Cu) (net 12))
 (segment (start 135.225 140.37) (end 136.37 140.37) (width 0.25) (layer F.Cu) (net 5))
 (segment (start 136.37 140.37) (end 137.5 141.5) (width 0.25) (layer F.Cu) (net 5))
 (segment (start 137.5 141.5) (end 138.15 141.5) (width 0.25) (layer F.Cu) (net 5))
 (segment (start 130.825 140.37) (end 129.506398 140.37) (width 0.25) (layer F.Cu) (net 10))
 (segment (start 128 137.5) (end 128.5 137) (width 0.25) (layer F.Cu) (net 10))
 (segment (start 128 138.863602) (end 128 137.5) (width 0.25) (layer F.Cu) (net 10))
 (segment (start 129.506398 140.37) (end 128 138.863602) (width 0.25) (layer F.Cu) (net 10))
 (segment (start 128.5 137) (end 129.15 137) (width 0.25) (layer F.Cu) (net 10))
 (segment (start 130.825 139.37) (end 130.825 138.825) (width 0.25) (layer F.Cu) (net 11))
 (segment (start 137.35 135.85) (end 137.35 137) (width 0.25) (layer F.Cu) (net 11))
 (segment (start 137 135.5) (end 137.35 135.85) (width 0.25) (layer F.Cu) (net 11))
 (segment (start 131 135.5) (end 137 135.5) (width 0.25) (layer F.Cu) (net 11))
 (segment (start 130.5 136) (end 131 135.5) (width 0.25) (layer F.Cu) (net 11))
 (segment (start 130.5 138.5) (end 130.5 136) (width 0.25) (layer F.Cu) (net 11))
 (segment (start 130.825 138.825) (end 130.5 138.5) (width 0.25) (layer F.Cu) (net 11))
 (segment (start 117.35 133.5) (end 118.54 133.5) (width 0.3048) (layer F.Cu) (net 21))
 (segment (start 118.54 133.5) (end 119.5 132.54) (width 0.3048) (layer F.Cu) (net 21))
 (segment (start 156 135.15) (end 156 133.96) (width 0.3048) (layer F.Cu) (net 14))
 (segment (start 156 133.96) (end 153.5 131.46) (width 0.3048) (layer F.Cu) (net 14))
 (segment (start 153.5 143.96) (end 154.89 143.96) (width 0.3048) (layer F.Cu) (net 15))
 (segment (start 154.89 143.96) (end 156 142.85) (width 0.3048) (layer F.Cu) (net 15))
 (segment (start 119.5 148.04) (end 117.04 148.04) (width 0.3048) (layer F.Cu) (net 17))
 (segment (start 114.65 145.65) (end 114.65 144.5) (width 0.3048) (layer F.Cu) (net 17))
 (segment (start 117.04 148.04) (end 114.65 145.65) (width 0.3048) (layer F.Cu) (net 17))
 (segment (start 119.5 130) (end 118 130) (width 0.3048) (layer B.Cu) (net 16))
 (segment (start 116.1 131.9) (end 116.1 140.7) (width 0.3048) (layer B.Cu) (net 16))
 (segment (start 118 130) (end 116.1 131.9) (width 0.3048) (layer B.Cu) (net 16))
 (segment (start 119.5 145.5) (end 117.6 145.5) (width 0.3048) (layer B.Cu) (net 16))
 (segment (start 117.4 139) (end 119.5 139) (width 0.3048) (layer B.Cu) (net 16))
 (segment (start 116.1 140.3) (end 117.4 139) (width 0.3048) (layer B.Cu) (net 16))
 (segment (start 116.1 144) (end 116.1 140.7) (width 0.3048) (layer B.Cu) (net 16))
 (segment (start 116.1 140.7) (end 116.1 140.3) (width 0.3048) (layer B.Cu) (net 16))
 (segment (start 117.6 145.5) (end 116.1 144) (width 0.3048) (layer B.Cu) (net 16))
 (segment (start 117.35 139.65) (end 118.85 139.65) (width 0.3048) (layer F.Cu) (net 16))
 (segment (start 118.85 139.65) (end 119.5 139) (width 0.3048) (layer F.Cu) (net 16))
 (segment (start 117.35 137.7) (end 118.8 137.7) (width 0.3048) (layer F.Cu) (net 19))
 (segment (start 118.8 137.7) (end 119.5 137) (width 0.3048) (layer F.Cu) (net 19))
 (segment (start 114.65 133.5) (end 114.8 133.5) (width 0.3048) (layer F.Cu) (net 22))
 (segment (start 114.8 133.5) (end 116.1 134.8) (width 0.3048) (layer F.Cu) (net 22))
 (segment (start 116.1 134.8) (end 116.1 143.25) (width 0.3048) (layer F.Cu) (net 22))
 (segment (start 116.1 143.25) (end 117.35 144.5) (width 0.3048) (layer F.Cu) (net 22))
 (segment (start 117.35 144.5) (end 117.35 144.15) (width 0.3048) (layer F.Cu) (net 22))
 (segment (start 117.35 144.15) (end 119.5 142) (width 0.3048) (layer F.Cu) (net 22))
 (segment (start 119.5 142) (end 119.5 141) (width 0.3048) (layer F.Cu) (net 22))
 (segment (start 136.5 147.5) (end 136.5 146.1) (width 0.3048) (layer B.Cu) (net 4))
 (segment (start 128.7 137) (end 126 137) (width 0.3048) (layer B.Cu) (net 4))
 (segment (start 130.2 138.5) (end 128.7 137) (width 0.3048) (layer B.Cu) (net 4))
 (segment (start 130.2 141.5) (end 130.2 138.5) (width 0.3048) (layer B.Cu) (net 4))
 (segment (start 131.8 143.1) (end 130.2 141.5) (width 0.3048) (layer B.Cu) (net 4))
 (segment (start 136.8 143.1) (end 131.8 143.1) (width 0.3048) (layer B.Cu) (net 4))
 (segment (start 137.3 143.6) (end 136.8 143.1) (width 0.3048) (layer B.Cu) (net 4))
 (segment (start 137.3 145.3) (end 137.3 143.6) (width 0.3048) (layer B.Cu) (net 4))
 (segment (start 136.5 146.1) (end 137.3 145.3) (width 0.3048) (layer B.Cu) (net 4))
 (segment (start 128.5 133.15) (end 128.5 134.5) (width 0.3048) (layer B.Cu) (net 4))
 (segment (start 128.5 134.5) (end 126 137) (width 0.3048) (layer B.Cu) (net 4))
 (segment (start 154 146.5) (end 153.5 146.5) (width 0.3048) (layer B.Cu) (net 13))
 (segment (start 153.5 134) (end 154 134) (width 0.3048) (layer B.Cu) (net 13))
 (segment (start 155.65 137.5) (end 156 137.85) (width 0.3048) (layer F.Cu) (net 23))
 (segment (start 156 140.15) (end 156 137.85) (width 0.3048) (layer F.Cu) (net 23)))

